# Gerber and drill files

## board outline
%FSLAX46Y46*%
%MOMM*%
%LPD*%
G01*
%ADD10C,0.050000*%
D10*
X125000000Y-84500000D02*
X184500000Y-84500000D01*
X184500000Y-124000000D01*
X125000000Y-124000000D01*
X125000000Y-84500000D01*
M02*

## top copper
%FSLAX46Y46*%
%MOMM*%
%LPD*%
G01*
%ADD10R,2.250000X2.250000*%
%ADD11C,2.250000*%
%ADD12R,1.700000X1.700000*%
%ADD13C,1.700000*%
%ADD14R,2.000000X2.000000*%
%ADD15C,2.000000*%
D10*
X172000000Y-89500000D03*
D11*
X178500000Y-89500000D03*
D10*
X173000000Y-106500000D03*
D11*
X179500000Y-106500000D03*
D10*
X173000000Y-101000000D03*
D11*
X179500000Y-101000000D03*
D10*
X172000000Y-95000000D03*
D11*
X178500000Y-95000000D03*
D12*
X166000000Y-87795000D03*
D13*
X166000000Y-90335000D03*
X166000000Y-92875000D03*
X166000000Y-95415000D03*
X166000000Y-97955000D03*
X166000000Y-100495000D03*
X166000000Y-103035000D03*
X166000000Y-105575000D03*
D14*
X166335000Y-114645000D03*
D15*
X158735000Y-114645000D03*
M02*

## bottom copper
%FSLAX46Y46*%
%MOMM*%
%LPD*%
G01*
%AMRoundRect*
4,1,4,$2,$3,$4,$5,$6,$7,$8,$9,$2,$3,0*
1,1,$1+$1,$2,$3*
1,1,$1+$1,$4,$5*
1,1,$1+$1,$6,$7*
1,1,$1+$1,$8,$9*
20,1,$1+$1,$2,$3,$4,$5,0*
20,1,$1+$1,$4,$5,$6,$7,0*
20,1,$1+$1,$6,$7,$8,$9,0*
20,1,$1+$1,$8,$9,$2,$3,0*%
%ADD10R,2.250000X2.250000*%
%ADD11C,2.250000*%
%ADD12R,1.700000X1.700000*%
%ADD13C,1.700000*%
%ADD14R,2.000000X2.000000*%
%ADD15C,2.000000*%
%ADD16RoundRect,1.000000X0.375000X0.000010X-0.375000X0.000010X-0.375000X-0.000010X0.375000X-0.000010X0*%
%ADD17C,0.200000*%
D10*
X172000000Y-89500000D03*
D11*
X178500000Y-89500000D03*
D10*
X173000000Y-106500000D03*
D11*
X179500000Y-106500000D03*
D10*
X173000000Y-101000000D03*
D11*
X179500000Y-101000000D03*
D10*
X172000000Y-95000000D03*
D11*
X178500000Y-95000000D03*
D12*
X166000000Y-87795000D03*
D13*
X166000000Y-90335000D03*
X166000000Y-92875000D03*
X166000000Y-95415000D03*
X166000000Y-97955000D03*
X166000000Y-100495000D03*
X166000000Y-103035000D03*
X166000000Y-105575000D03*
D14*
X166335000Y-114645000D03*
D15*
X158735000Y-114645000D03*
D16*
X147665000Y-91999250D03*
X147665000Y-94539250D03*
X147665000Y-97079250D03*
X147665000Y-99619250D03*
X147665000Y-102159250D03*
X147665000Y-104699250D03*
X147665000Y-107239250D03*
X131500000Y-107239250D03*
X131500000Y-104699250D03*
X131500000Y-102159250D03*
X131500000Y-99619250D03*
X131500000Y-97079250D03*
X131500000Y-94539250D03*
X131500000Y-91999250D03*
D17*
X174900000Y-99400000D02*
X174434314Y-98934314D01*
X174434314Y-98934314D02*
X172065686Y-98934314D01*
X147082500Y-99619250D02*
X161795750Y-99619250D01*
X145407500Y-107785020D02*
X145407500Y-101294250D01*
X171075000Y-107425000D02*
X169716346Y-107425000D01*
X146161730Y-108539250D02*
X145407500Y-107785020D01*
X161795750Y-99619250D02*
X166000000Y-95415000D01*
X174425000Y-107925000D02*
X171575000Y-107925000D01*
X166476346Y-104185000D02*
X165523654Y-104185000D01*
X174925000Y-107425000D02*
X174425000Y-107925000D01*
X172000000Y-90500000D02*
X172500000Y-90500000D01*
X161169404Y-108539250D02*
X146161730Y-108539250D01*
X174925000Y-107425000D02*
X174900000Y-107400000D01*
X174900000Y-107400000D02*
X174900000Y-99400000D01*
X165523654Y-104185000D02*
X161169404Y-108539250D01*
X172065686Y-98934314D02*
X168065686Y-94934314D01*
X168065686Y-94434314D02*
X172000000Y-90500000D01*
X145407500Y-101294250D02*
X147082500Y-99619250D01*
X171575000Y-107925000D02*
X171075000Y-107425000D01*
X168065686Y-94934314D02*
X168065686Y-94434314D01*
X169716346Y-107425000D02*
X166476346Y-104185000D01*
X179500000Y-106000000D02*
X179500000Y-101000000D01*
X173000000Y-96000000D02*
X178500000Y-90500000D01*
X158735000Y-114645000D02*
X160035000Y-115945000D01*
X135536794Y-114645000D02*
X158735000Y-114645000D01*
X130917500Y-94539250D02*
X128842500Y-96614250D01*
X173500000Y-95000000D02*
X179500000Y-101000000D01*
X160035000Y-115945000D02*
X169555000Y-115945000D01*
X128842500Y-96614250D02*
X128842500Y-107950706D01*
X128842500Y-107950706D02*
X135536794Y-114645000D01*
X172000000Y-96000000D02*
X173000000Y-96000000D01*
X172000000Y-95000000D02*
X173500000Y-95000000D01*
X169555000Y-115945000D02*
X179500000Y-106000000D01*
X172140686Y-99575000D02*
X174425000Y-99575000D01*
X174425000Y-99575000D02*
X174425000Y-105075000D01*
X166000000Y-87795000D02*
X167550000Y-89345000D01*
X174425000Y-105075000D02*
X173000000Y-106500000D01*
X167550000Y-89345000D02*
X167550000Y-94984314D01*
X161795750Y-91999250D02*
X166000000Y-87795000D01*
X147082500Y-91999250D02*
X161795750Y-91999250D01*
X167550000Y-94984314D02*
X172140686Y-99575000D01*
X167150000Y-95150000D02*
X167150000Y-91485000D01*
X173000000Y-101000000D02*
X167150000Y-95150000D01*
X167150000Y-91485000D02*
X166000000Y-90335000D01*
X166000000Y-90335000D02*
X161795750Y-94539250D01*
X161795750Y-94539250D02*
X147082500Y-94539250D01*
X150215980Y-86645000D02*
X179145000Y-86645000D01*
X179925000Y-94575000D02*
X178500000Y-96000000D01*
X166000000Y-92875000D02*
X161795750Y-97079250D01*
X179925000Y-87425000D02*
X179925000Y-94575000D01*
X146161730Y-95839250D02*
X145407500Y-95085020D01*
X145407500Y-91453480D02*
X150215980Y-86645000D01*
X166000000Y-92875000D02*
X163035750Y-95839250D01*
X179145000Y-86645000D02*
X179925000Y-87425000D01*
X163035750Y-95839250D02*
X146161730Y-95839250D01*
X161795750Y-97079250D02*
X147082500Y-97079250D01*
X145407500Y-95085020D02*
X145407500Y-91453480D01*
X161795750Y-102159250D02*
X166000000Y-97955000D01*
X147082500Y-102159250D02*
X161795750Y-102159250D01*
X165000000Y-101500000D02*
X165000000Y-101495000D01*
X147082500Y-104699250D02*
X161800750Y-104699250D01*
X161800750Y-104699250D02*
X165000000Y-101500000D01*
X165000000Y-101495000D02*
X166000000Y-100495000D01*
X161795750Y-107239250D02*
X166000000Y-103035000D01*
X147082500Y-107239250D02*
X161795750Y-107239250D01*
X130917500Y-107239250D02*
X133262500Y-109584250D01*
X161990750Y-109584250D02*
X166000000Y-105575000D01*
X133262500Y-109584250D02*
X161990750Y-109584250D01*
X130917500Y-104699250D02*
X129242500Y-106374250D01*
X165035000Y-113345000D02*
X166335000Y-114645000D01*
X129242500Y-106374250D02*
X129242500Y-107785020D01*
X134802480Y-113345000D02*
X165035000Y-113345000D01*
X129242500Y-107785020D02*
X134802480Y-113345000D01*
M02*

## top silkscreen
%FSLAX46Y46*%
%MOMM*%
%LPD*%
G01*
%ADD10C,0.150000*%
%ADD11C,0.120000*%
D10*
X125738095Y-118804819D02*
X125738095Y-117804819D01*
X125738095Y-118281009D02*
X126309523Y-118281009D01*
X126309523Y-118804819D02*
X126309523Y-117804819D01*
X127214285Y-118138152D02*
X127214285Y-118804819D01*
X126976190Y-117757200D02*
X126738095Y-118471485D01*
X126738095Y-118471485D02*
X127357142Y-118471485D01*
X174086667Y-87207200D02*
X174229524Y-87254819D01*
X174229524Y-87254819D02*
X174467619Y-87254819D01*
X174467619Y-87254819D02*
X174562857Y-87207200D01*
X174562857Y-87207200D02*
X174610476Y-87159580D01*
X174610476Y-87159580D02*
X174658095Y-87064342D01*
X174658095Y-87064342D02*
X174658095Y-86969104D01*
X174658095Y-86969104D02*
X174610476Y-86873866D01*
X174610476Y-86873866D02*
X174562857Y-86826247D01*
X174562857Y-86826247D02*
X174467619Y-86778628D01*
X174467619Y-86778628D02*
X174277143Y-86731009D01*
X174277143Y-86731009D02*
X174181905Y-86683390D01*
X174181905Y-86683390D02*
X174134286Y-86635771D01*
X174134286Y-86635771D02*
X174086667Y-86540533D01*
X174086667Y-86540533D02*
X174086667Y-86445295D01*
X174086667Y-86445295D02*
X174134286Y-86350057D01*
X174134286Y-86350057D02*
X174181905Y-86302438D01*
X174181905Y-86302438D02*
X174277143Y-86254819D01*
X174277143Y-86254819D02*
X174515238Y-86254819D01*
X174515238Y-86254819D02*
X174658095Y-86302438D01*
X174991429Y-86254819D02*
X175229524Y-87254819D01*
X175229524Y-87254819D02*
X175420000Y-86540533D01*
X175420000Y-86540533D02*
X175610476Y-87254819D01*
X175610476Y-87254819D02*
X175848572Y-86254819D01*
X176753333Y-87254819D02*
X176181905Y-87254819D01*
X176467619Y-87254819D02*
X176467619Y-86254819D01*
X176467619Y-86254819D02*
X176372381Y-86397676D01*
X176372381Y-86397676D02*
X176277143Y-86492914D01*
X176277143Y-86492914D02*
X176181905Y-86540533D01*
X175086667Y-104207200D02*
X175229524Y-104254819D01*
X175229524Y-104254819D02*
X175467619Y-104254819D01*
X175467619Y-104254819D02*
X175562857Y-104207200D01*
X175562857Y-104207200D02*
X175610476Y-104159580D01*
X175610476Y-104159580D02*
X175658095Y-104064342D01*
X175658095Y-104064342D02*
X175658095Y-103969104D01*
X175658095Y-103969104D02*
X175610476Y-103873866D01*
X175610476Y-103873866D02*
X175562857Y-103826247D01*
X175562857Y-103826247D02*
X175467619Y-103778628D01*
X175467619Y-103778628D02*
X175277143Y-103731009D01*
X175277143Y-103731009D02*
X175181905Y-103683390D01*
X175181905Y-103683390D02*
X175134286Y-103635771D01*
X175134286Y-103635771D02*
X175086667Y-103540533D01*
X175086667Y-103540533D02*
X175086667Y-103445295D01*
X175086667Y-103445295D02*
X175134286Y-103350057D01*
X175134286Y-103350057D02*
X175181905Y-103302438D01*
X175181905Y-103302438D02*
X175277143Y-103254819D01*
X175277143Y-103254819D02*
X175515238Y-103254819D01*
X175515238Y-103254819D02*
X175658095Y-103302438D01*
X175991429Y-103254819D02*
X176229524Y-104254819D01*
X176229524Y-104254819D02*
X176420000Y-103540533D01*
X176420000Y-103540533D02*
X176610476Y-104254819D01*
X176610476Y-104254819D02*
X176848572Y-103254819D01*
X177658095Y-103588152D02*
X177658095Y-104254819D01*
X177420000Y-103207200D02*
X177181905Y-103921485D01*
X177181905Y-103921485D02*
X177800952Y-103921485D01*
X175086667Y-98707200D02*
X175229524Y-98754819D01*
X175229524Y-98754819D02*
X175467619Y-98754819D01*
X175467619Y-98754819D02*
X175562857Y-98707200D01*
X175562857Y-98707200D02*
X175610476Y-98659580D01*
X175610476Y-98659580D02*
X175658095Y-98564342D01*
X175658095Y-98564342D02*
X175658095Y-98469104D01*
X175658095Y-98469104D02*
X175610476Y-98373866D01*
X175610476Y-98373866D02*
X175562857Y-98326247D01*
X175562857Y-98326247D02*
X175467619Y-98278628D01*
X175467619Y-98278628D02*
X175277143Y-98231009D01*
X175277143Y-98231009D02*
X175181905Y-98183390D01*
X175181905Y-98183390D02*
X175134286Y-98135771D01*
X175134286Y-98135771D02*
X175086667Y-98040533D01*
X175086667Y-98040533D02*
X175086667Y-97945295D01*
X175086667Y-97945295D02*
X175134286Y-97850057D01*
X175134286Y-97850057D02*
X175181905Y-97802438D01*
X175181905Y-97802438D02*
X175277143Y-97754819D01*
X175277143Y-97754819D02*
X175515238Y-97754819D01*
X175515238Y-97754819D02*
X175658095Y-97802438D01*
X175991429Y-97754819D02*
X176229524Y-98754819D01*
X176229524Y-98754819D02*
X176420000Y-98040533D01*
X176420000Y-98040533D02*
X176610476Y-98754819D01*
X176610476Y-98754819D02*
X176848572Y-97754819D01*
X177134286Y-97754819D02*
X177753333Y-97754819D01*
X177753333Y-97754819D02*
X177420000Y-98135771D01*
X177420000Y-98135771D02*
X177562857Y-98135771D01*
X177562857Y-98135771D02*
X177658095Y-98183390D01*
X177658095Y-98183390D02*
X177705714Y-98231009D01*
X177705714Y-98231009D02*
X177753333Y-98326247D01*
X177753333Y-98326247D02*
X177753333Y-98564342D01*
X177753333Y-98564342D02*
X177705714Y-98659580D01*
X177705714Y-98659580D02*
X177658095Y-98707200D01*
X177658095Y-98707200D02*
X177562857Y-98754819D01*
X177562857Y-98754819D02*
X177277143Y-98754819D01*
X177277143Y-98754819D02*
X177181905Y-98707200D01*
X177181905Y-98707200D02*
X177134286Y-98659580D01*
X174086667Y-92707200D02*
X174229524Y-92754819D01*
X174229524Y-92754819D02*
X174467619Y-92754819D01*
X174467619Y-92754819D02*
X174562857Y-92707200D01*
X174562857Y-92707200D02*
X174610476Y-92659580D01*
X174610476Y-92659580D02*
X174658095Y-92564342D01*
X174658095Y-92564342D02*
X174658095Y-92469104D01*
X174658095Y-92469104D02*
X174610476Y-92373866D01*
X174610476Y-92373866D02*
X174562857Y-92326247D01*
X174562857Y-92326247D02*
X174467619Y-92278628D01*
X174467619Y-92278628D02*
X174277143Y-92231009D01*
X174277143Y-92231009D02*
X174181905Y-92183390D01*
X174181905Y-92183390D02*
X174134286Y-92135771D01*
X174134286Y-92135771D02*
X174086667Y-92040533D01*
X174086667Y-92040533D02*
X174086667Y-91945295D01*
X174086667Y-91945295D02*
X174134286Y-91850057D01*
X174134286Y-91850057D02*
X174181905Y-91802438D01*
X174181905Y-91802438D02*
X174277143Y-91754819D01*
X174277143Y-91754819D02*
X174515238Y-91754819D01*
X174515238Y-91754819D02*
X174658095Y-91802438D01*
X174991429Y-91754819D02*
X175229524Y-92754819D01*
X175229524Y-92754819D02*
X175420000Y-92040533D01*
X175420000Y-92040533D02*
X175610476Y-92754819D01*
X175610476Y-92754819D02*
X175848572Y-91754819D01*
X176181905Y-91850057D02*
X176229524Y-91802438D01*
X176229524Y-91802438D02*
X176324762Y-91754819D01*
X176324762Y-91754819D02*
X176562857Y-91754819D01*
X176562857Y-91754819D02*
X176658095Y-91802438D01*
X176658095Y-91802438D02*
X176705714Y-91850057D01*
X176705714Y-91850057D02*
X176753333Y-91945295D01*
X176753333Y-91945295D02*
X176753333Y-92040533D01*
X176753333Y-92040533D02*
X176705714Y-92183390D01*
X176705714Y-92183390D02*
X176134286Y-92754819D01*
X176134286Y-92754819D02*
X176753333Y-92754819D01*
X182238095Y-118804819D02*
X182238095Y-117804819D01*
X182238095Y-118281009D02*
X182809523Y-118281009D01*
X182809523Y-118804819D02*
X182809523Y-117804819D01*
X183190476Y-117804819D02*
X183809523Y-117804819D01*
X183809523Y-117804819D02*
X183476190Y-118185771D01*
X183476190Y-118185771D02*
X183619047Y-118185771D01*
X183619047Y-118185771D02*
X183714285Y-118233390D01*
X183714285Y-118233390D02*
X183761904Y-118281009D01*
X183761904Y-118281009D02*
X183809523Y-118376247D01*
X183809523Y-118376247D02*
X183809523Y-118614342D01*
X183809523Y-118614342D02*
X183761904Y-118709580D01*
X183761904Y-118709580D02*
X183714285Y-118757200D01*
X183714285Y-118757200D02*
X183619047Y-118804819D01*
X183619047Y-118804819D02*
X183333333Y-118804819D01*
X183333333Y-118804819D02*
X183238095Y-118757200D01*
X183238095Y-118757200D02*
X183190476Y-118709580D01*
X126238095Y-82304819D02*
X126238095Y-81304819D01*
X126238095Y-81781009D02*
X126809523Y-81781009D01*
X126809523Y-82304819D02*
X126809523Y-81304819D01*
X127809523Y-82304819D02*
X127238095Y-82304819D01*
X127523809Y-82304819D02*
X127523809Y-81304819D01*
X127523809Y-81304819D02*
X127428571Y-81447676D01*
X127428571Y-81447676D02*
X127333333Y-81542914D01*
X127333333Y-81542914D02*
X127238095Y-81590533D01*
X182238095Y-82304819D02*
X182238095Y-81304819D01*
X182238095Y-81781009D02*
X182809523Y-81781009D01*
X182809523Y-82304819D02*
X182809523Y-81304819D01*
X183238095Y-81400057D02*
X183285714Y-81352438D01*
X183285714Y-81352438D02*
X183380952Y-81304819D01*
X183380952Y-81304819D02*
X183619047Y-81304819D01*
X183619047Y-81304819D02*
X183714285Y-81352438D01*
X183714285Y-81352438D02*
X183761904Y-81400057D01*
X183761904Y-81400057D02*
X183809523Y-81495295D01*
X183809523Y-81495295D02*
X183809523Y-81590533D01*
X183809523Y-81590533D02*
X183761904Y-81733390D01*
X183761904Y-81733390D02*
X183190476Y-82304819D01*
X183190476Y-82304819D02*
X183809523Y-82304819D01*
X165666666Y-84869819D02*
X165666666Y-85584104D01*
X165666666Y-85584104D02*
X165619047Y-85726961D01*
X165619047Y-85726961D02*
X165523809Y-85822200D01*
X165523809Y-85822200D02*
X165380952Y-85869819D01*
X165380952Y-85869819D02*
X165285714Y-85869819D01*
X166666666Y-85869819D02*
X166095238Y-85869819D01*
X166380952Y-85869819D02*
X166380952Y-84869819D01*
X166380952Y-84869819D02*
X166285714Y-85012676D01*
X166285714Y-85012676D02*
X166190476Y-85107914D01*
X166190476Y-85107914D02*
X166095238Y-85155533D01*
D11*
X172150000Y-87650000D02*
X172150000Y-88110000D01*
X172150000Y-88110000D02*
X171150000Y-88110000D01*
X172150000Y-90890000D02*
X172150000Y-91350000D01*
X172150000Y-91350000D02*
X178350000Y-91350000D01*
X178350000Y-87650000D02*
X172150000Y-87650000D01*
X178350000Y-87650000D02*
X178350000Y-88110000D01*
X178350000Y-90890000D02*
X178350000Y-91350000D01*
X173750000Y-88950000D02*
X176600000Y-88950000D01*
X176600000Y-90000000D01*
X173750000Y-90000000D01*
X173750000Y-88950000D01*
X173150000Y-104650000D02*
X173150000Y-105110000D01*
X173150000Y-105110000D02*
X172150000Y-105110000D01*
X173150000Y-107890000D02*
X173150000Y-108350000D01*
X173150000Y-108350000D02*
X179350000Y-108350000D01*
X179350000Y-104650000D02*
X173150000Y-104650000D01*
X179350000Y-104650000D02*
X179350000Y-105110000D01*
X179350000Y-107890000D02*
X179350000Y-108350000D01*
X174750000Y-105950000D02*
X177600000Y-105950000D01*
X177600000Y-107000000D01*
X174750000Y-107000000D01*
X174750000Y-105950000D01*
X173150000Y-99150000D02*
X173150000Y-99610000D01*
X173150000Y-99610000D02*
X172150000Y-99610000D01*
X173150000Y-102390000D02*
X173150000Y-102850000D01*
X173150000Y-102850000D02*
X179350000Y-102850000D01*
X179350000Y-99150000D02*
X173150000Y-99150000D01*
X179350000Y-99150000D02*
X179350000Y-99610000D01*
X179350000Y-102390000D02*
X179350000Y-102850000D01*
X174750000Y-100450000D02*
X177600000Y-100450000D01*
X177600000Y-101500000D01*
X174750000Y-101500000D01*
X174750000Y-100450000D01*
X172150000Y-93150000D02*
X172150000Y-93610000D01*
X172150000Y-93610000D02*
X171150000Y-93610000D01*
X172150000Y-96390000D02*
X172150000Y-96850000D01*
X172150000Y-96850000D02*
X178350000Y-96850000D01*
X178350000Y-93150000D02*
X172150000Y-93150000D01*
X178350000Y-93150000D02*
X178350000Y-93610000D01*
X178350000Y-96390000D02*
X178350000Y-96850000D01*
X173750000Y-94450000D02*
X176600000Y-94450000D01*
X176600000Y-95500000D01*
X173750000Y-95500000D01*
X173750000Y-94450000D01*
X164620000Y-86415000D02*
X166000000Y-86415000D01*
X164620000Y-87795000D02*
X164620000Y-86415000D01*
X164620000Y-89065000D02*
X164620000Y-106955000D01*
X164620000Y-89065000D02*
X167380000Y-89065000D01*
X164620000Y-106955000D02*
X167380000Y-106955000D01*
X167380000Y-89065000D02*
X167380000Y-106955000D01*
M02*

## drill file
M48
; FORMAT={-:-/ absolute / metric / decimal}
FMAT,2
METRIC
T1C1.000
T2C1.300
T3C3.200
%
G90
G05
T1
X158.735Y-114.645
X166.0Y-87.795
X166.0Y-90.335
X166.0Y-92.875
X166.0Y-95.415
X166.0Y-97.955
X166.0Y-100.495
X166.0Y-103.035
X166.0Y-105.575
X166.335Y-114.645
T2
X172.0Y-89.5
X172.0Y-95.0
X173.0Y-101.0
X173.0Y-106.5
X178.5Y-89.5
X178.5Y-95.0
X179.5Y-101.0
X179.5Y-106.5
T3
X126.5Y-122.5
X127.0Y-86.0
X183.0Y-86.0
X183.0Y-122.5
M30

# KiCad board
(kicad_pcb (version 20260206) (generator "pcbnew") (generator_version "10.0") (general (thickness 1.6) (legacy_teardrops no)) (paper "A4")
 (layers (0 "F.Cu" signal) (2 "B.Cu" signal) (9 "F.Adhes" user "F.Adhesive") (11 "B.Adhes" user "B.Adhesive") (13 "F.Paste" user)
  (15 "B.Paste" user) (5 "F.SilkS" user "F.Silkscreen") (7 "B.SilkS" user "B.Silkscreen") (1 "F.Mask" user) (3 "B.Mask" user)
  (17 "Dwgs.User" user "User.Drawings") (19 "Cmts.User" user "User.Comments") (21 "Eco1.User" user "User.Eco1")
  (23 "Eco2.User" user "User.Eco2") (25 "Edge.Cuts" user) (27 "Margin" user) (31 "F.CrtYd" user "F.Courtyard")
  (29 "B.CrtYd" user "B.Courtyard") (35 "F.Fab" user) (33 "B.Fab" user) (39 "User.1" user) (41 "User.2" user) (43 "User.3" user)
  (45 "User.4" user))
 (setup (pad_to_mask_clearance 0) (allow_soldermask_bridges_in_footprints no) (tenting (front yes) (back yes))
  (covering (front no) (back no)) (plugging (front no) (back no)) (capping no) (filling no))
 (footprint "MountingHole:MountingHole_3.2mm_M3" (layer "F.Cu") (at 126.5 122.5)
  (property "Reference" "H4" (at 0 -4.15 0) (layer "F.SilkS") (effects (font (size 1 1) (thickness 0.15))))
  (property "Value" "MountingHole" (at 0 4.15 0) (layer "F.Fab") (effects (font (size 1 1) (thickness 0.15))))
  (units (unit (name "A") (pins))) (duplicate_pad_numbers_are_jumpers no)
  (pad "" np_thru_hole circle (at 0 0) (size 3.2 3.2) (drill 3.2) (layers "*.Cu" "*.Mask")))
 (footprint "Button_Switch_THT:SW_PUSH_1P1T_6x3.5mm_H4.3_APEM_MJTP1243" (layer "F.Cu") (at 172 89.5)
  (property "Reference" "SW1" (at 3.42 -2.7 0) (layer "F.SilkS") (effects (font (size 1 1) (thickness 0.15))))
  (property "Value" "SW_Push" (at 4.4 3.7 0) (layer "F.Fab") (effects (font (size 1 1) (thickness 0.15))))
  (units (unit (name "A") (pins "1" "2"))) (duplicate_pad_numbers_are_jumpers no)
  (fp_line (start 0.15 -1.85) (end 0.15 -1.39) (stroke (width 0.12) (type default)) (layer "F.SilkS"))
  (fp_line (start 0.15 -1.39) (end -0.85 -1.39) (stroke (width 0.12) (type default)) (layer "F.SilkS"))
  (fp_line (start 0.15 1.39) (end 0.15 1.85) (stroke (width 0.12) (type solid)) (layer "F.SilkS"))
  (fp_line (start 0.15 1.85) (end 6.35 1.85) (stroke (width 0.12) (type solid)) (layer "F.SilkS"))
  (fp_line (start 6.35 -1.85) (end 0.15 -1.85) (stroke (width 0.12) (type solid)) (layer "F.SilkS"))
  (fp_line (start 6.35 -1.85) (end 6.35 -1.39) (stroke (width 0.12) (type solid)) (layer "F.SilkS"))
  (fp_line (start 6.35 1.39) (end 6.35 1.85) (stroke (width 0.12) (type solid)) (layer "F.SilkS"))
  (fp_rect (start 1.75 -0.55) (end 4.6 0.5) (stroke (width 0.12) (type default)) (fill no) (layer "F.SilkS"))
  (pad "1" thru_hole rect (at 0 0 90) (size 2.25 2.25) (drill 1.3) (layers "*.Cu" "*.Mask") (remove_unused_layers no) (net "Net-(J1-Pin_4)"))
  (pad "2" thru_hole circle (at 6.5 0 90) (size 2.25 2.25) (drill 1.3) (layers "*.Cu" "*.Mask") (remove_unused_layers no) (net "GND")))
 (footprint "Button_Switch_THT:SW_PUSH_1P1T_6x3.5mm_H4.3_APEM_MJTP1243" (layer "F.Cu") (at 173 106.5)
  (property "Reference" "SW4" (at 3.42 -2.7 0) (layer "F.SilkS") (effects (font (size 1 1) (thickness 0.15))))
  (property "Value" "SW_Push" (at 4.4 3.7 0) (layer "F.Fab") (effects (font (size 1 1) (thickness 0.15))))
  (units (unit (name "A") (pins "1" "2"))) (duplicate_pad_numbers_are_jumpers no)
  (fp_line (start 0.15 -1.85) (end 0.15 -1.39) (stroke (width 0.12) (type default)) (layer "F.SilkS"))
  (fp_line (start 0.15 -1.39) (end -0.85 -1.39) (stroke (width 0.12) (type default)) (layer "F.SilkS"))
  (fp_line (start 0.15 1.39) (end 0.15 1.85) (stroke (width 0.12) (type solid)) (layer "F.SilkS"))
  (fp_line (start 0.15 1.85) (end 6.35 1.85) (stroke (width 0.12) (type solid)) (layer "F.SilkS"))
  (fp_line (start 6.35 -1.85) (end 0.15 -1.85) (stroke (width 0.12) (type solid)) (layer "F.SilkS"))
  (fp_line (start 6.35 -1.85) (end 6.35 -1.39) (stroke (width 0.12) (type solid)) (layer "F.SilkS"))
  (fp_line (start 6.35 1.39) (end 6.35 1.85) (stroke (width 0.12) (type solid)) (layer "F.SilkS"))
  (fp_rect (start 1.75 -0.55) (end 4.6 0.5) (stroke (width 0.12) (type default)) (fill no) (layer "F.SilkS"))
  (pad "1" thru_hole rect (at 0 0 90) (size 2.25 2.25) (drill 1.3) (layers "*.Cu" "*.Mask") (remove_unused_layers no) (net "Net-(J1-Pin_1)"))
  (pad "2" thru_hole circle (at 6.5 0 90) (size 2.25 2.25) (drill 1.3) (layers "*.Cu" "*.Mask") (remove_unused_layers no) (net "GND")))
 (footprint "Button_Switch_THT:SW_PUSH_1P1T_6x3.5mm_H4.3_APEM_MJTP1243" (layer "F.Cu") (at 173 101)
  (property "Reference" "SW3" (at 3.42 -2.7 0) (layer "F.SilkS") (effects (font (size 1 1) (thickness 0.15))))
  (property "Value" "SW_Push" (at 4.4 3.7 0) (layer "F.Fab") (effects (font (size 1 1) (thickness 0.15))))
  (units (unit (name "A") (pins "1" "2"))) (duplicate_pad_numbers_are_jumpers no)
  (fp_line (start 0.15 -1.85) (end 0.15 -1.39) (stroke (width 0.12) (type default)) (layer "F.SilkS"))
  (fp_line (start 0.15 -1.39) (end -0.85 -1.39) (stroke (width 0.12) (type default)) (layer "F.SilkS"))
  (fp_line (start 0.15 1.39) (end 0.15 1.85) (stroke (width 0.12) (type solid)) (layer "F.SilkS"))
  (fp_line (start 0.15 1.85) (end 6.35 1.85) (stroke (width 0.12) (type solid)) (layer "F.SilkS"))
  (fp_line (start 6.35 -1.85) (end 0.15 -1.85) (stroke (width 0.12) (type solid)) (layer "F.SilkS"))
  (fp_line (start 6.35 -1.85) (end 6.35 -1.39) (stroke (width 0.12) (type solid)) (layer "F.SilkS"))
  (fp_line (start 6.35 1.39) (end 6.35 1.85) (stroke (width 0.12) (type solid)) (layer "F.SilkS"))
  (fp_rect (start 1.75 -0.55) (end 4.6 0.5) (stroke (width 0.12) (type default)) (fill no) (layer "F.SilkS"))
  (pad "1" thru_hole rect (at 0 0 90) (size 2.25 2.25) (drill 1.3) (layers "*.Cu" "*.Mask") (remove_unused_layers no) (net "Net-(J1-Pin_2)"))
  (pad "2" thru_hole circle (at 6.5 0 90) (size 2.25 2.25) (drill 1.3) (layers "*.Cu" "*.Mask") (remove_unused_layers no) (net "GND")))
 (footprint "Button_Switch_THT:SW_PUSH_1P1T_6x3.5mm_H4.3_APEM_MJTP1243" (layer "F.Cu") (at 172 95)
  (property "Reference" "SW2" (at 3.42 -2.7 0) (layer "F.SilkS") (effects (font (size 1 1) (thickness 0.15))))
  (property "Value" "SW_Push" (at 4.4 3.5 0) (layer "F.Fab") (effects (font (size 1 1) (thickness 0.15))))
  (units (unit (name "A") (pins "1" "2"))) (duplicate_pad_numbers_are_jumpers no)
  (fp_line (start 0.15 -1.85) (end 0.15 -1.39) (stroke (width 0.12) (type default)) (layer "F.SilkS"))
  (fp_line (start 0.15 -1.39) (end -0.85 -1.39) (stroke (width 0.12) (type default)) (layer "F.SilkS"))
  (fp_line (start 0.15 1.39) (end 0.15 1.85) (stroke (width 0.12) (type solid)) (layer "F.SilkS"))
  (fp_line (start 0.15 1.85) (end 6.35 1.85) (stroke (width 0.12) (type solid)) (layer "F.SilkS"))
  (fp_line (start 6.35 -1.85) (end 0.15 -1.85) (stroke (width 0.12) (type solid)) (layer "F.SilkS"))
  (fp_line (start 6.35 -1.85) (end 6.35 -1.39) (stroke (width 0.12) (type solid)) (layer "F.SilkS"))
  (fp_line (start 6.35 1.39) (end 6.35 1.85) (stroke (width 0.12) (type solid)) (layer "F.SilkS"))
  (fp_rect (start 1.75 -0.55) (end 4.6 0.5) (stroke (width 0.12) (type default)) (fill no) (layer "F.SilkS"))
  (pad "1" thru_hole rect (at 0 0 90) (size 2.25 2.25) (drill 1.3) (layers "*.Cu" "*.Mask") (remove_unused_layers no) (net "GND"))
  (pad "2" thru_hole circle (at 6.5 0 90) (size 2.25 2.25) (drill 1.3) (layers "*.Cu" "*.Mask") (remove_unused_layers no)
   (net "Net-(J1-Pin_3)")))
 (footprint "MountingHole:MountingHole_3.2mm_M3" (layer "F.Cu") (at 183 122.5)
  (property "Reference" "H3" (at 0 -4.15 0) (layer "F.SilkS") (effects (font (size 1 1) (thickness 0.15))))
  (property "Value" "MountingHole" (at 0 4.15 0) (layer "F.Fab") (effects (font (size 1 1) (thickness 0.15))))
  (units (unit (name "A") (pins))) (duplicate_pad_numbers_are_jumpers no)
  (pad "" np_thru_hole circle (at 0 0) (size 3.2 3.2) (drill 3.2) (layers "*.Cu" "*.Mask")))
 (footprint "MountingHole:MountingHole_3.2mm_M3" (layer "F.Cu") (at 127 86)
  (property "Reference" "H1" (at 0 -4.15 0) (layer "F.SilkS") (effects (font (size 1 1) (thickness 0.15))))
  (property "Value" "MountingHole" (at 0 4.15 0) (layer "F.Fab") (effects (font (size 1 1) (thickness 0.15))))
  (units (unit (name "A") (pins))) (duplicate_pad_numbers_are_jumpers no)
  (pad "" np_thru_hole circle (at 0 0) (size 3.2 3.2) (drill 3.2) (layers "*.Cu" "*.Mask")))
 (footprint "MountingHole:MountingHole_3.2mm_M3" (layer "F.Cu") (at 183 86)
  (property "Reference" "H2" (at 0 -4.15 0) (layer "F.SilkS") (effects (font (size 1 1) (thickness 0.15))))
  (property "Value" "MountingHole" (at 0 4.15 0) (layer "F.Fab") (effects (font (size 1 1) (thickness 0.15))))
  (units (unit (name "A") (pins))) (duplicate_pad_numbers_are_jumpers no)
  (pad "" np_thru_hole circle (at 0 0) (size 3.2 3.2) (drill 3.2) (layers "*.Cu" "*.Mask")))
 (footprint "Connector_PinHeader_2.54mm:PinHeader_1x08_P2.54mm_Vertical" (layer "F.Cu") (at 166 87.795)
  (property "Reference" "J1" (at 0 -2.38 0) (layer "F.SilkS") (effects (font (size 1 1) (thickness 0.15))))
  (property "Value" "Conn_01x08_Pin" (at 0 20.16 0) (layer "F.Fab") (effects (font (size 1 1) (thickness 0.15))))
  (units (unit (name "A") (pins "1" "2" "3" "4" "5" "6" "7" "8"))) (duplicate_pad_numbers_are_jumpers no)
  (fp_line (start -1.38 -1.38) (end 0 -1.38) (stroke (width 0.12) (type solid)) (layer "F.SilkS"))
  (fp_line (start -1.38 0) (end -1.38 -1.38) (stroke (width 0.12) (type solid)) (layer "F.SilkS"))
  (fp_line (start -1.38 1.27) (end -1.38 19.16) (stroke (width 0.12) (type solid)) (layer "F.SilkS"))
  (fp_line (start -1.38 1.27) (end 1.38 1.27) (stroke (width 0.12) (type solid)) (layer "F.SilkS"))
  (fp_line (start -1.38 19.16) (end 1.38 19.16) (stroke (width 0.12) (type solid)) (layer "F.SilkS"))
  (fp_line (start 1.38 1.27) (end 1.38 19.16) (stroke (width 0.12) (type solid)) (layer "F.SilkS"))
  (pad "1" thru_hole rect (at 0 0) (size 1.7 1.7) (drill 1) (layers "*.Cu" "*.Mask") (remove_unused_layers no) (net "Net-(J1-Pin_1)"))
  (pad "2" thru_hole circle (at 0 2.54) (size 1.7 1.7) (drill 1) (layers "*.Cu" "*.Mask") (remove_unused_layers no) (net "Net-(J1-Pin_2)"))
  (pad "3" thru_hole circle (at 0 5.08) (size 1.7 1.7) (drill 1) (layers "*.Cu" "*.Mask") (remove_unused_layers no) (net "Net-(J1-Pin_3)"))
  (pad "4" thru_hole circle (at 0 7.62) (size 1.7 1.7) (drill 1) (layers "*.Cu" "*.Mask") (remove_unused_layers no) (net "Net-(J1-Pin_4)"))
  (pad "5" thru_hole circle (at 0 10.16) (size 1.7 1.7) (drill 1) (layers "*.Cu" "*.Mask") (remove_unused_layers no) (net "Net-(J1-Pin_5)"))
  (pad "6" thru_hole circle (at 0 12.7) (size 1.7 1.7) (drill 1) (layers "*.Cu" "*.Mask") (remove_unused_layers no) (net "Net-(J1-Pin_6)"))
  (pad "7" thru_hole circle (at 0 15.24) (size 1.7 1.7) (drill 1) (layers "*.Cu" "*.Mask") (remove_unused_layers no) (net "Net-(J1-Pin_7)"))
  (pad "8" thru_hole circle (at 0 17.78) (size 1.7 1.7) (drill 1) (layers "*.Cu" "*.Mask") (remove_unused_layers no) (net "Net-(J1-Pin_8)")))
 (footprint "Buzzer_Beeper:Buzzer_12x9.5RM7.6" (layer "B.Cu") (at 166.335 114.645 180)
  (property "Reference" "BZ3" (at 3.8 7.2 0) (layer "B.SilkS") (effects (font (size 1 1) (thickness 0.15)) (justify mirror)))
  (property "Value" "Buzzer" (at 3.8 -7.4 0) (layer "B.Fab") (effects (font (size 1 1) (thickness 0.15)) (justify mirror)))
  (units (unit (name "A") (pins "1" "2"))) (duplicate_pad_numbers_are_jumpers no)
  (pad "1" thru_hole rect (at 0 0 180) (size 2 2) (drill 1) (layers "*.Cu" "*.Mask") (remove_unused_layers no) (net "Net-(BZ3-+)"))
  (pad "2" thru_hole circle (at 7.6 0 180) (size 2 2) (drill 1) (layers "*.Cu" "*.Mask") (remove_unused_layers no) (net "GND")))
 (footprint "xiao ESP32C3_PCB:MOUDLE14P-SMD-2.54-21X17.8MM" (layer "B.Cu") (at 148.5 110.11925 180)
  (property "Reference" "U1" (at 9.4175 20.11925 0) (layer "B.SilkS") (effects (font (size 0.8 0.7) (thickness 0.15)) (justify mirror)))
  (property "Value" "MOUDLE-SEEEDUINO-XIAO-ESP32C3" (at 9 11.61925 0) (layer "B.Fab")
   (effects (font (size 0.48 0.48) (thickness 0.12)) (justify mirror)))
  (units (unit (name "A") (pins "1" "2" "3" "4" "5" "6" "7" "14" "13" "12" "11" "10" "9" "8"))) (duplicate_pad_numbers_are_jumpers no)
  (pad "1" smd roundrect (at 0.835 18.12 180) (size 2.75 2) (layers "B.Cu" "B.Mask" "B.Paste") (roundrect_rratio 0.5) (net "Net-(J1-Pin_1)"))
  (pad "2" smd roundrect (at 0.835 15.58 180) (size 2.75 2) (layers "B.Cu" "B.Mask" "B.Paste") (roundrect_rratio 0.5) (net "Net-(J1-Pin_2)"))
  (pad "3" smd roundrect (at 0.835 13.04 180) (size 2.75 2) (layers "B.Cu" "B.Mask" "B.Paste") (roundrect_rratio 0.5) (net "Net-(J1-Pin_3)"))
  (pad "4" smd roundrect (at 0.835 10.5 180) (size 2.75 2) (layers "B.Cu" "B.Mask" "B.Paste") (roundrect_rratio 0.5) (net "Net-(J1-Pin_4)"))
  (pad "5" smd roundrect (at 0.835 7.96 180) (size 2.75 2) (layers "B.Cu" "B.Mask" "B.Paste") (roundrect_rratio 0.5) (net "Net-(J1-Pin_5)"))
  (pad "6" smd roundrect (at 0.835 5.42 180) (size 2.75 2) (layers "B.Cu" "B.Mask" "B.Paste") (roundrect_rratio 0.5) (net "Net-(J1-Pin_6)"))
  (pad "7" smd roundrect (at 0.835 2.88 180) (size 2.75 2) (layers "B.Cu" "B.Mask" "B.Paste") (roundrect_rratio 0.5) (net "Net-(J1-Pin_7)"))
  (pad "8" smd roundrect (at 17 2.88 180) (size 2.75 2) (layers "B.Cu" "B.Mask" "B.Paste") (roundrect_rratio 0.5) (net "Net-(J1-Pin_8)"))
  (pad "9" smd roundrect (at 17 5.42 180) (size 2.75 2) (layers "B.Cu" "B.Mask" "B.Paste") (roundrect_rratio 0.5) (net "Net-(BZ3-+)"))
  (pad "10" smd roundrect (at 17 7.96 180) (size 2.75 2) (layers "B.Cu" "B.Mask" "B.Paste") (roundrect_rratio 0.5)
   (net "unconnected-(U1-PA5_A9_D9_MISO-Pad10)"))
  (pad "11" smd roundrect (at 17 10.5 180) (size 2.75 2) (layers "B.Cu" "B.Mask" "B.Paste") (roundrect_rratio 0.5)
   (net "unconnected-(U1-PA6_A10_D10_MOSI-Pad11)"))
  (pad "12" smd roundrect (at 17 13.04 180) (size 2.75 2) (layers "B.Cu" "B.Mask" "B.Paste") (roundrect_rratio 0.5) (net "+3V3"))
  (pad "13" smd roundrect (at 17 15.58 180) (size 2.75 2) (layers "B.Cu" "B.Mask" "B.Paste") (roundrect_rratio 0.5) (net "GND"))
  (pad "14" smd roundrect (at 17 18.12 180) (size 2.75 2) (layers "B.Cu" "B.Mask" "B.Paste") (roundrect_rratio 0.5)
   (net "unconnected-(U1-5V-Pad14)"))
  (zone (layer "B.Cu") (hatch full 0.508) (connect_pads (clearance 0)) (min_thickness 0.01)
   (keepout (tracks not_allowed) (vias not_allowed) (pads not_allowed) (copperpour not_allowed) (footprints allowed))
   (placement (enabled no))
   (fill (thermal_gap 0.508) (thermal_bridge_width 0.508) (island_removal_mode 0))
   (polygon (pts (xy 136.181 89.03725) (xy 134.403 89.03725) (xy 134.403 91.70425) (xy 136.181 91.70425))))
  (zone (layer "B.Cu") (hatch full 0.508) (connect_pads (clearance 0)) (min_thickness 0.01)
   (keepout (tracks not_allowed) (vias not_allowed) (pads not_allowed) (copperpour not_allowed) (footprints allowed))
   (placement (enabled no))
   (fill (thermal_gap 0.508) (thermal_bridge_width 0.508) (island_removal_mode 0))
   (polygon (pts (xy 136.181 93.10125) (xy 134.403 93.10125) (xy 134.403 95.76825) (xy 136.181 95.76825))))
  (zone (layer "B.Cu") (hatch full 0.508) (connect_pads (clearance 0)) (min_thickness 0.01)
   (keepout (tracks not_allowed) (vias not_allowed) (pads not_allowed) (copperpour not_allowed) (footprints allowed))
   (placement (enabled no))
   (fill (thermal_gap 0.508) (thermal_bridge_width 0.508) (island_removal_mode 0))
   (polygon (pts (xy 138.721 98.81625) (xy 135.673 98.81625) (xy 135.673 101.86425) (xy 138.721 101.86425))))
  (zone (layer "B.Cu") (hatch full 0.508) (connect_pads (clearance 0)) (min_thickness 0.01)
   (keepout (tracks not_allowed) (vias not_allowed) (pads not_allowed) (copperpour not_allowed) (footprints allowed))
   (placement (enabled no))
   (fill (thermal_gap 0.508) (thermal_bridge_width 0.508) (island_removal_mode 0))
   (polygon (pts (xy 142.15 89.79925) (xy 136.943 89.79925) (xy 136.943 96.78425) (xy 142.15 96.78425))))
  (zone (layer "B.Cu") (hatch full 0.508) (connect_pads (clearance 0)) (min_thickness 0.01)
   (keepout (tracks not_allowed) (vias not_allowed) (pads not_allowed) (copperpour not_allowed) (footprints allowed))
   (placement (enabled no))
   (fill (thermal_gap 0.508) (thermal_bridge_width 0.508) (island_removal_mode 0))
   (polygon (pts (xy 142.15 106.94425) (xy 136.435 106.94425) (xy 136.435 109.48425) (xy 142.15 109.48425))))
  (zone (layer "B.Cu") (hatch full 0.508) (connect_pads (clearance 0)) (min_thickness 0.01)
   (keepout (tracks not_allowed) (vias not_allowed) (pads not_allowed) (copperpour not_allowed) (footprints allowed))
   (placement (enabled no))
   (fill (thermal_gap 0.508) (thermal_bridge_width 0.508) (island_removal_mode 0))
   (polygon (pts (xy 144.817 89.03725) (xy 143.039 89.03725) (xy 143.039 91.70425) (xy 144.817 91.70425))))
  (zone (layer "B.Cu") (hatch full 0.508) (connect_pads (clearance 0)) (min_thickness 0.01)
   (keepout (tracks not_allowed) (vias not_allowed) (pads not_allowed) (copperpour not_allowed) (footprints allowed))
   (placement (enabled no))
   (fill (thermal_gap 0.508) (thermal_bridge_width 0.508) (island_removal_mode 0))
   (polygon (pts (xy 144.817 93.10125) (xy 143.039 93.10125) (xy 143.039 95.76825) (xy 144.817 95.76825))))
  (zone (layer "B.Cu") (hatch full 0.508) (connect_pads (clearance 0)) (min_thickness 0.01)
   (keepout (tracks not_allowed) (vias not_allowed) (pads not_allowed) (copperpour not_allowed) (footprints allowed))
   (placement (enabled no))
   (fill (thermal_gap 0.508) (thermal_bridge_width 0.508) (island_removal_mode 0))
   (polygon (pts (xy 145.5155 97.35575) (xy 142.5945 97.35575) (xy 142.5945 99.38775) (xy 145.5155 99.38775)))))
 (gr_rect (start 125 84.5) (end 184.5 124) (stroke (width 0.05) (type solid)) (fill no) (layer "Edge.Cuts"))
 (segment (start 174.9 99.4) (end 174.434314 98.934314) (width 0.2) (layer "B.Cu") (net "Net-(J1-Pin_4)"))
 (segment (start 174.434314 98.934314) (end 172.065686 98.934314) (width 0.2) (layer "B.Cu") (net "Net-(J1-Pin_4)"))
 (segment (start 147.0825 99.61925) (end 161.79575 99.61925) (width 0.2) (layer "B.Cu") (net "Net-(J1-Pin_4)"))
 (segment (start 145.4075 107.78502) (end 145.4075 101.29425) (width 0.2) (layer "B.Cu") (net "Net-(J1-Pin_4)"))
 (segment (start 171.075 107.425) (end 169.716346 107.425) (width 0.2) (layer "B.Cu") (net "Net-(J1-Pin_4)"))
 (segment (start 146.16173 108.53925) (end 145.4075 107.78502) (width 0.2) (layer "B.Cu") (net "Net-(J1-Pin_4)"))
 (segment (start 161.79575 99.61925) (end 166 95.415) (width 0.2) (layer "B.Cu") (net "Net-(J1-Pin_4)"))
 (segment (start 174.425 107.925) (end 171.575 107.925) (width 0.2) (layer "B.Cu") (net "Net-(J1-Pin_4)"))
 (segment (start 166.476346 104.185) (end 165.523654 104.185) (width 0.2) (layer "B.Cu") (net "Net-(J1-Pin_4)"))
 (segment (start 174.925 107.425) (end 174.425 107.925) (width 0.2) (layer "B.Cu") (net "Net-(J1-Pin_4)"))
 (segment (start 172 90.5) (end 172.5 90.5) (width 0.2) (layer "B.Cu") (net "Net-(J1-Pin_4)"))
 (segment (start 161.169404 108.53925) (end 146.16173 108.53925) (width 0.2) (layer "B.Cu") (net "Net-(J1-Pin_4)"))
 (segment (start 174.925 107.425) (end 174.9 107.4) (width 0.2) (layer "B.Cu") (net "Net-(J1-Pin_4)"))
 (segment (start 174.9 107.4) (end 174.9 99.4) (width 0.2) (layer "B.Cu") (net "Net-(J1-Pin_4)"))
 (segment (start 165.523654 104.185) (end 161.169404 108.53925) (width 0.2) (layer "B.Cu") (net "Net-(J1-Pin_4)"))
 (segment (start 172.065686 98.934314) (end 168.065686 94.934314) (width 0.2) (layer "B.Cu") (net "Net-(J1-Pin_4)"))
 (segment (start 168.065686 94.434314) (end 172 90.5) (width 0.2) (layer "B.Cu") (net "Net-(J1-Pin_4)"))
 (segment (start 145.4075 101.29425) (end 147.0825 99.61925) (width 0.2) (layer "B.Cu") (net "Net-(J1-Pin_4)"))
 (segment (start 171.575 107.925) (end 171.075 107.425) (width 0.2) (layer "B.Cu") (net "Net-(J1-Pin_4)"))
 (segment (start 168.065686 94.934314) (end 168.065686 94.434314) (width 0.2) (layer "B.Cu") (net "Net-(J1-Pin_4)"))
 (segment (start 169.716346 107.425) (end 166.476346 104.185) (width 0.2) (layer "B.Cu") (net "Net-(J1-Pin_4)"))
 (segment (start 179.5 106) (end 179.5 101) (width 0.2) (layer "B.Cu") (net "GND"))
 (segment (start 173 96) (end 178.5 90.5) (width 0.2) (layer "B.Cu") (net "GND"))
 (segment (start 158.735 114.645) (end 160.035 115.945) (width 0.2) (layer "B.Cu") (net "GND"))
 (segment (start 135.536794 114.645) (end 158.735 114.645) (width 0.2) (layer "B.Cu") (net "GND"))
 (segment (start 130.9175 94.53925) (end 128.8425 96.61425) (width 0.2) (layer "B.Cu") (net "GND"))
 (segment (start 173.5 95) (end 179.5 101) (width 0.2) (layer "B.Cu") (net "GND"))
 (segment (start 160.035 115.945) (end 169.555 115.945) (width 0.2) (layer "B.Cu") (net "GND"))
 (segment (start 128.8425 96.61425) (end 128.8425 107.950706) (width 0.2) (layer "B.Cu") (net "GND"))
 (segment (start 128.8425 107.950706) (end 135.536794 114.645) (width 0.2) (layer "B.Cu") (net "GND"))
 (segment (start 172 96) (end 173 96) (width 0.2) (layer "B.Cu") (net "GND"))
 (segment (start 172 95) (end 173.5 95) (width 0.2) (layer "B.Cu") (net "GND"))
 (segment (start 169.555 115.945) (end 179.5 106) (width 0.2) (layer "B.Cu") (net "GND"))
 (segment (start 172.140686 99.575) (end 174.425 99.575) (width 0.2) (layer "B.Cu") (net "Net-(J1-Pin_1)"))
 (segment (start 174.425 99.575) (end 174.425 105.075) (width 0.2) (layer "B.Cu") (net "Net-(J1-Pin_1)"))
 (segment (start 166 87.795) (end 167.55 89.345) (width 0.2) (layer "B.Cu") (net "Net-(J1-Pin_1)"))
 (segment (start 174.425 105.075) (end 173 106.5) (width 0.2) (layer "B.Cu") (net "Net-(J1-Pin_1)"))
 (segment (start 167.55 89.345) (end 167.55 94.984314) (width 0.2) (layer "B.Cu") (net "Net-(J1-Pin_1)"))
 (segment (start 161.79575 91.99925) (end 166 87.795) (width 0.2) (layer "B.Cu") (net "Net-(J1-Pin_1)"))
 (segment (start 147.0825 91.99925) (end 161.79575 91.99925) (width 0.2) (layer "B.Cu") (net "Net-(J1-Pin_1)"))
 (segment (start 167.55 94.984314) (end 172.140686 99.575) (width 0.2) (layer "B.Cu") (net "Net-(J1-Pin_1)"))
 (segment (start 167.15 95.15) (end 167.15 91.485) (width 0.2) (layer "B.Cu") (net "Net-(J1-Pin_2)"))
 (segment (start 173 101) (end 167.15 95.15) (width 0.2) (layer "B.Cu") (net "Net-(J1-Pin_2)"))
 (segment (start 167.15 91.485) (end 166 90.335) (width 0.2) (layer "B.Cu") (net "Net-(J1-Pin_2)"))
 (segment (start 166 90.335) (end 161.79575 94.53925) (width 0.2) (layer "B.Cu") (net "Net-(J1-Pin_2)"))
 (segment (start 161.79575 94.53925) (end 147.0825 94.53925) (width 0.2) (layer "B.Cu") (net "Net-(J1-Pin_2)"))
 (segment (start 150.21598 86.645) (end 179.145 86.645) (width 0.2) (layer "B.Cu") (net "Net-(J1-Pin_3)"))
 (segment (start 179.925 94.575) (end 178.5 96) (width 0.2) (layer "B.Cu") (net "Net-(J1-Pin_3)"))
 (segment (start 166 92.875) (end 161.79575 97.07925) (width 0.2) (layer "B.Cu") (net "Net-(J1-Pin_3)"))
 (segment (start 179.925 87.425) (end 179.925 94.575) (width 0.2) (layer "B.Cu") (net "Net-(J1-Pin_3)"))
 (segment (start 146.16173 95.83925) (end 145.4075 95.08502) (width 0.2) (layer "B.Cu") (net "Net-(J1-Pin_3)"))
 (segment (start 145.4075 91.45348) (end 150.21598 86.645) (width 0.2) (layer "B.Cu") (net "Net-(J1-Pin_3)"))
 (segment (start 166 92.875) (end 163.03575 95.83925) (width 0.2) (layer "B.Cu") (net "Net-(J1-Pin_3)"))
 (segment (start 179.145 86.645) (end 179.925 87.425) (width 0.2) (layer "B.Cu") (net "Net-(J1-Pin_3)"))
 (segment (start 163.03575 95.83925) (end 146.16173 95.83925) (width 0.2) (layer "B.Cu") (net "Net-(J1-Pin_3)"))
 (segment (start 161.79575 97.07925) (end 147.0825 97.07925) (width 0.2) (layer "B.Cu") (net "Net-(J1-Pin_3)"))
 (segment (start 145.4075 95.08502) (end 145.4075 91.45348) (width 0.2) (layer "B.Cu") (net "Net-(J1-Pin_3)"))
 (segment (start 161.79575 102.15925) (end 166 97.955) (width 0.2) (layer "B.Cu") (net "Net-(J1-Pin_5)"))
 (segment (start 147.0825 102.15925) (end 161.79575 102.15925) (width 0.2) (layer "B.Cu") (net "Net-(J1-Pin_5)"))
 (segment (start 165 101.5) (end 165 101.495) (width 0.2) (layer "B.Cu") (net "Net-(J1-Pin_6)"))
 (segment (start 147.0825 104.69925) (end 161.80075 104.69925) (width 0.2) (layer "B.Cu") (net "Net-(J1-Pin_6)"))
 (segment (start 161.80075 104.69925) (end 165 101.5) (width 0.2) (layer "B.Cu") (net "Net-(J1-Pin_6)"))
 (segment (start 165 101.495) (end 166 100.495) (width 0.2) (layer "B.Cu") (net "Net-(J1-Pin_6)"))
 (segment (start 161.79575 107.23925) (end 166 103.035) (width 0.2) (layer "B.Cu") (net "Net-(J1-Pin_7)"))
 (segment (start 147.0825 107.23925) (end 161.79575 107.23925) (width 0.2) (layer "B.Cu") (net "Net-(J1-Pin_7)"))
 (segment (start 130.9175 107.23925) (end 133.2625 109.58425) (width 0.2) (layer "B.Cu") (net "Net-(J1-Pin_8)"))
 (segment (start 161.99075 109.58425) (end 166 105.575) (width 0.2) (layer "B.Cu") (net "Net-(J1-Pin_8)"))
 (segment (start 133.2625 109.58425) (end 161.99075 109.58425) (width 0.2) (layer "B.Cu") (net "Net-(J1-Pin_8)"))
 (segment (start 130.9175 104.69925) (end 129.2425 106.37425) (width 0.2) (layer "B.Cu") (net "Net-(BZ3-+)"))
 (segment (start 165.035 113.345) (end 166.335 114.645) (width 0.2) (layer "B.Cu") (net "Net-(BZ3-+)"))
 (segment (start 129.2425 106.37425) (end 129.2425 107.78502) (width 0.2) (layer "B.Cu") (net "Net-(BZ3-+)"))
 (segment (start 134.80248 113.345) (end 165.035 113.345) (width 0.2) (layer "B.Cu") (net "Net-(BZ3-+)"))
 (segment (start 129.2425 107.78502) (end 134.80248 113.345) (width 0.2) (layer "B.Cu") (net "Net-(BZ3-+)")))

